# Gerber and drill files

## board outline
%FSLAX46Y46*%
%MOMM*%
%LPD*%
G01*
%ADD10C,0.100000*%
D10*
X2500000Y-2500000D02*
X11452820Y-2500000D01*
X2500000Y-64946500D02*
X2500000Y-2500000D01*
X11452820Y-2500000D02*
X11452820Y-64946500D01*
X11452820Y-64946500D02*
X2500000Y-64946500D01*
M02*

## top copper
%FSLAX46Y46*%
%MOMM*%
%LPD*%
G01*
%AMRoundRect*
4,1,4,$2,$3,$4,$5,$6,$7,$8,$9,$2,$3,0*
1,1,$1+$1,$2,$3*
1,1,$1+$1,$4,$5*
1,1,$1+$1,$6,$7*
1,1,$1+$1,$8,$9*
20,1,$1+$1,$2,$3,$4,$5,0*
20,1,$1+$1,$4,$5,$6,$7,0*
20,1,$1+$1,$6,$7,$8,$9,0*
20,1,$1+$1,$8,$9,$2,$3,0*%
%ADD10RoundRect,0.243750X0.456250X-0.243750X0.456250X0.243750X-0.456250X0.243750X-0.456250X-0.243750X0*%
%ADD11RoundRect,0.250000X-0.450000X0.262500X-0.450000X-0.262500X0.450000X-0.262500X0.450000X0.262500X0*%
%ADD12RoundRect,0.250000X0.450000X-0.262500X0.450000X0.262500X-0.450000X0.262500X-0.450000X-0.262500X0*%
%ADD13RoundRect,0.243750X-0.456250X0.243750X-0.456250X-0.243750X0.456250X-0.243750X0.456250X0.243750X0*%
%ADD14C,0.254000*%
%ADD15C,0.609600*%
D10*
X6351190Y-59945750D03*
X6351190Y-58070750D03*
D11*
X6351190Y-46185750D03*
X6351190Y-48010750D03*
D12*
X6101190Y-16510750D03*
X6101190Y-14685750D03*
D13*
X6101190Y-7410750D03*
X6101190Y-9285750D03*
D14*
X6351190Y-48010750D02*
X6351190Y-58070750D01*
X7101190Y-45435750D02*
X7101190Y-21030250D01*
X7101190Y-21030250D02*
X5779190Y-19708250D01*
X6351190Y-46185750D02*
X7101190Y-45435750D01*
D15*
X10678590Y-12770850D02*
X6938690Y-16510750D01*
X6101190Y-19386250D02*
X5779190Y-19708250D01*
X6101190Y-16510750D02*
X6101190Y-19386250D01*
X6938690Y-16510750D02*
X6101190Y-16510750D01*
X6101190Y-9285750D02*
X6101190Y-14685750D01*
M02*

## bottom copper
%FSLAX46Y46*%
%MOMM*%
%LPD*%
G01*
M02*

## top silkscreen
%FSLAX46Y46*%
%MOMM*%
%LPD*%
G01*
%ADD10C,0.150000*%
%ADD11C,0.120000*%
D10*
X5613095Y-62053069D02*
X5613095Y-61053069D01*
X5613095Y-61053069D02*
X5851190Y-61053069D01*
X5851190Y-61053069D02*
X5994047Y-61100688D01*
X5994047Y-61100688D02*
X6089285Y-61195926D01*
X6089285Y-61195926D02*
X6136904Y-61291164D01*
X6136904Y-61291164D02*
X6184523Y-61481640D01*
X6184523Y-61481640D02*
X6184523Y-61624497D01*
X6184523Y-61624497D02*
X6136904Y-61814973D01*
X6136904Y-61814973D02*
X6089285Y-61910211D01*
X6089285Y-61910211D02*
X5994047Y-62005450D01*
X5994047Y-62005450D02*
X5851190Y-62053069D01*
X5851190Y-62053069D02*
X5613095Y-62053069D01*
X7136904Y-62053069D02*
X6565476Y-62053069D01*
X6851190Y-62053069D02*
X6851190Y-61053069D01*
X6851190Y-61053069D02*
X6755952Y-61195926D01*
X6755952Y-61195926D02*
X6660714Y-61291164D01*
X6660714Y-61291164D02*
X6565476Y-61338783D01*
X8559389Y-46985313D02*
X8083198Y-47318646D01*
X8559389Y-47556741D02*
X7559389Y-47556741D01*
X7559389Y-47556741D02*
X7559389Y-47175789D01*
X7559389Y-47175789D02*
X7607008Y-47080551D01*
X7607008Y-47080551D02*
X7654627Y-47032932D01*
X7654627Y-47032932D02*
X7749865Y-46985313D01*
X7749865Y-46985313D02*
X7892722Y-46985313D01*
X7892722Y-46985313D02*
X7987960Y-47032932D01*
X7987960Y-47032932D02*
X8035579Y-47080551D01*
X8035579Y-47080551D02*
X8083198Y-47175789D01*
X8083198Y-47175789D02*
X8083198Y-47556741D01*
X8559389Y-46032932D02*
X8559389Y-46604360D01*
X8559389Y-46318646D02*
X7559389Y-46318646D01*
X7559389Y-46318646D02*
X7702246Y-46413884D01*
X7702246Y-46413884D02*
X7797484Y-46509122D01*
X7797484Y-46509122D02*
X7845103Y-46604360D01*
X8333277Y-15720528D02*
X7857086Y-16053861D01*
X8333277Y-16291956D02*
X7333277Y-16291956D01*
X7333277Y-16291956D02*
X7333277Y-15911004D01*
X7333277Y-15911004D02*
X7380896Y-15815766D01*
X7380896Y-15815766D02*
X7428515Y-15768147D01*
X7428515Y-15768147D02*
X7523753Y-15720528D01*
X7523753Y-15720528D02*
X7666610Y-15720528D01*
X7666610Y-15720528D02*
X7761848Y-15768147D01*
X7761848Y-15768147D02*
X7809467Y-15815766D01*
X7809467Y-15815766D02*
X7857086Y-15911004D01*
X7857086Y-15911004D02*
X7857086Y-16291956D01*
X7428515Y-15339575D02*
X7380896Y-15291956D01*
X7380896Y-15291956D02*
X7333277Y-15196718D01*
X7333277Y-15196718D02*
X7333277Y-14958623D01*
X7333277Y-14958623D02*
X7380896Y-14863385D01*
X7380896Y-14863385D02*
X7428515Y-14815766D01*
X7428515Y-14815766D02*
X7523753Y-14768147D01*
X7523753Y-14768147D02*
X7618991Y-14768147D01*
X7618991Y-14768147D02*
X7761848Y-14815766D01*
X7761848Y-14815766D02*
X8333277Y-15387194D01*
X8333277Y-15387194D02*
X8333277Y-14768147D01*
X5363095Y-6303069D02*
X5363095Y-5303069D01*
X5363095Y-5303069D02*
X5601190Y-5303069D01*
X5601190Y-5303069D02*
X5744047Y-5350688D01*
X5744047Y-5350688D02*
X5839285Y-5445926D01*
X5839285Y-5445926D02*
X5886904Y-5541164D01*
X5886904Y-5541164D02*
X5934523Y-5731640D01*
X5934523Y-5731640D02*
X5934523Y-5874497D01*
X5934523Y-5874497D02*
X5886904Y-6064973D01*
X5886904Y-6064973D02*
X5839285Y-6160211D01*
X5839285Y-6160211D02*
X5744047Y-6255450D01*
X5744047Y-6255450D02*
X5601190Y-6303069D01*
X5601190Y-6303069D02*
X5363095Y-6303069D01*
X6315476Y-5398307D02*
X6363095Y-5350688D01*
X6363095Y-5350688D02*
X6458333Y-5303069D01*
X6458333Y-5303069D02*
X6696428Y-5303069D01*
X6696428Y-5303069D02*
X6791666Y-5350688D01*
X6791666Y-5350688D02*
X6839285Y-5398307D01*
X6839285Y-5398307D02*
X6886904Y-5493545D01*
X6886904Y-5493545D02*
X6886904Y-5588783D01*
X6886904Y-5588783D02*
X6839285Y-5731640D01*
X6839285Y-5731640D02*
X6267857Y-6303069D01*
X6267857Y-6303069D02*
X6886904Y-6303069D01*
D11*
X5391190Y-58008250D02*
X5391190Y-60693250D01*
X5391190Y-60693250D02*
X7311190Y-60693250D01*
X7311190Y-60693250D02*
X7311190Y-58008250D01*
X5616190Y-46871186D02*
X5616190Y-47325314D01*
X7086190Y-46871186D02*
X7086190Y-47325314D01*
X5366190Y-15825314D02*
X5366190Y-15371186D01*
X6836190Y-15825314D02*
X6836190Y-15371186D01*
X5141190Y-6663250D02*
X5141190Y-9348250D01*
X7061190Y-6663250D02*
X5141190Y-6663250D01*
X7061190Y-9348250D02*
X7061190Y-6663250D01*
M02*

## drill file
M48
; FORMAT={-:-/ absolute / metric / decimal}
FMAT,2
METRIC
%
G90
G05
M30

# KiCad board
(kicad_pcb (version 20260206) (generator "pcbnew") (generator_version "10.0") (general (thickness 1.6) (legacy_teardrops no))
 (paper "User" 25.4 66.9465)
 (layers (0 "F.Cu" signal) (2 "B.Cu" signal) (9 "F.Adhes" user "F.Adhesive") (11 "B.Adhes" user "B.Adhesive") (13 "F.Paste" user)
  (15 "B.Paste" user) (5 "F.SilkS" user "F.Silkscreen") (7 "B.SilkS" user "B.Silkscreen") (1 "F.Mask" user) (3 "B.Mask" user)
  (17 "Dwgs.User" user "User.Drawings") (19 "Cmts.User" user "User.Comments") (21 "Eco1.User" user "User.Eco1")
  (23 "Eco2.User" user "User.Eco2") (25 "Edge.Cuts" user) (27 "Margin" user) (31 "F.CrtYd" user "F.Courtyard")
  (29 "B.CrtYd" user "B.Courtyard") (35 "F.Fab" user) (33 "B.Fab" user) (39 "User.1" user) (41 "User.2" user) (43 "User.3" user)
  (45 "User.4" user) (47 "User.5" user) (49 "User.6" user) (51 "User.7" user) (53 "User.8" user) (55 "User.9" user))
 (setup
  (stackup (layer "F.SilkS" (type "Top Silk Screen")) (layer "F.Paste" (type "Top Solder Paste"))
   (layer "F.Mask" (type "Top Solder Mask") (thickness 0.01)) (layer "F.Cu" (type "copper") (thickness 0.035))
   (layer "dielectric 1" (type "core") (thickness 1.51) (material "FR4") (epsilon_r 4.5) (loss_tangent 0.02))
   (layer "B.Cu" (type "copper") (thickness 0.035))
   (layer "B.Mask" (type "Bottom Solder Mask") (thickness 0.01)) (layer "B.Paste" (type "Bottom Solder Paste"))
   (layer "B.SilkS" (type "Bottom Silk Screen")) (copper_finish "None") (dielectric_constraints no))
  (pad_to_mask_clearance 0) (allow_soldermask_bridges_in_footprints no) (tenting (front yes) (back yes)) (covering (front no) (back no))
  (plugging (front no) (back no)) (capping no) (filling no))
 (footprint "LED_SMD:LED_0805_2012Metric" (layer "F.Cu") (at 6.35119 59.00825 90)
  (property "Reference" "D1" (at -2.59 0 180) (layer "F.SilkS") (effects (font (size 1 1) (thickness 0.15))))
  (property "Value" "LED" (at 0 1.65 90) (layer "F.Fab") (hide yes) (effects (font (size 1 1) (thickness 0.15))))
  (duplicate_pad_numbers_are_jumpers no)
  (fp_line (start 1 -0.96) (end -1.685 -0.96) (stroke (width 0.12) (type solid)) (layer "F.SilkS"))
  (fp_line (start -1.685 -0.96) (end -1.685 0.96) (stroke (width 0.12) (type solid)) (layer "F.SilkS"))
  (fp_line (start -1.685 0.96) (end 1 0.96) (stroke (width 0.12) (type solid)) (layer "F.SilkS"))
  (pad "1" smd roundrect (at -0.9375 0 90) (size 0.975 1.4) (layers "F.Cu" "F.Mask" "F.Paste") (roundrect_rratio 0.25) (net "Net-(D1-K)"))
  (pad "2" smd roundrect (at 0.9375 0 90) (size 0.975 1.4) (layers "F.Cu" "F.Mask" "F.Paste") (roundrect_rratio 0.25) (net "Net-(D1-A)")))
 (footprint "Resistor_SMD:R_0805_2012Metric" (layer "F.Cu") (at 6.35119 47.09825 -90)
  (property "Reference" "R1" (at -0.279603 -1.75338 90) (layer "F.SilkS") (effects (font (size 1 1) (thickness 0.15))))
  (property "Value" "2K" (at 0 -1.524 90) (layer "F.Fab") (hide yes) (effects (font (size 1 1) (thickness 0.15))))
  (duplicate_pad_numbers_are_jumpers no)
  (fp_line (start -0.227064 0.735) (end 0.227064 0.735) (stroke (width 0.12) (type solid)) (layer "F.SilkS"))
  (fp_line (start -0.227064 -0.735) (end 0.227064 -0.735) (stroke (width 0.12) (type solid)) (layer "F.SilkS"))
  (pad "1" smd roundrect (at -0.9125 0 270) (size 1.025 1.4) (layers "F.Cu" "F.Mask" "F.Paste") (roundrect_rratio 0.243902439) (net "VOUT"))
  (pad "2" smd roundrect (at 0.9125 0 270) (size 1.025 1.4) (layers "F.Cu" "F.Mask" "F.Paste") (roundrect_rratio 0.243902439)
   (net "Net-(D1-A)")))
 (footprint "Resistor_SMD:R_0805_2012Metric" (layer "F.Cu") (at 6.10119 15.59825 90)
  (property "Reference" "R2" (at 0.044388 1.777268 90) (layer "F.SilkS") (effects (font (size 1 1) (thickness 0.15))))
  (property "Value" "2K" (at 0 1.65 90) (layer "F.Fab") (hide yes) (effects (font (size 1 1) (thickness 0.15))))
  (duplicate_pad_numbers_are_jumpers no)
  (fp_line (start -0.227064 -0.735) (end 0.227064 -0.735) (stroke (width 0.12) (type solid)) (layer "F.SilkS"))
  (fp_line (start -0.227064 0.735) (end 0.227064 0.735) (stroke (width 0.12) (type solid)) (layer "F.SilkS"))
  (pad "1" smd roundrect (at -0.9125 0 90) (size 1.025 1.4) (layers "F.Cu" "F.Mask" "F.Paste") (roundrect_rratio 0.243902439) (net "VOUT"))
  (pad "2" smd roundrect (at 0.9125 0 90) (size 1.025 1.4) (layers "F.Cu" "F.Mask" "F.Paste") (roundrect_rratio 0.243902439)
   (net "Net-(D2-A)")))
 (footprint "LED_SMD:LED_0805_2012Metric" (layer "F.Cu") (at 6.10119 8.34825 -90)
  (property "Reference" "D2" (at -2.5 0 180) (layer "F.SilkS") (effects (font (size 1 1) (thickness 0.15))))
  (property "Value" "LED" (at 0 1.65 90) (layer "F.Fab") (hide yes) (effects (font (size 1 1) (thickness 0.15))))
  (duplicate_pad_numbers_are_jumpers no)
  (fp_line (start -1.685 0.96) (end 1 0.96) (stroke (width 0.12) (type solid)) (layer "F.SilkS"))
  (fp_line (start -1.685 -0.96) (end -1.685 0.96) (stroke (width 0.12) (type solid)) (layer "F.SilkS"))
  (fp_line (start 1 -0.96) (end -1.685 -0.96) (stroke (width 0.12) (type solid)) (layer "F.SilkS"))
  (pad "1" smd roundrect (at -0.9375 0 270) (size 0.975 1.4) (layers "F.Cu" "F.Mask" "F.Paste") (roundrect_rratio 0.25) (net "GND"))
  (pad "2" smd roundrect (at 0.9375 0 270) (size 0.975 1.4) (layers "F.Cu" "F.Mask" "F.Paste") (roundrect_rratio 0.25) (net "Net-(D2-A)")))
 (gr_line (start 2.5 2.5) (end 11.45282 2.5) (stroke (width 0.1) (type default)) (layer "Edge.Cuts"))
 (gr_line (start 2.5 64.9465) (end 2.5 2.5) (stroke (width 0.1) (type default)) (layer "Edge.Cuts"))
 (gr_line (start 11.45282 2.5) (end 11.45282 64.9465) (stroke (width 0.1) (type default)) (layer "Edge.Cuts"))
 (gr_line (start 11.45282 64.9465) (end 2.5 64.9465) (stroke (width 0.1) (type default)) (layer "Edge.Cuts"))
 (segment (start 6.35119 48.01075) (end 6.35119 58.07075) (width 0.254) (layer "F.Cu") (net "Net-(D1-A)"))
 (segment (start 7.10119 45.43575) (end 7.10119 21.03025) (width 0.254) (layer "F.Cu") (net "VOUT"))
 (segment (start 7.10119 21.03025) (end 5.77919 19.70825) (width 0.254) (layer "F.Cu") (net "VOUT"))
 (segment (start 6.35119 46.18575) (end 7.10119 45.43575) (width 0.254) (layer "F.Cu") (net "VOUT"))
 (segment (start 10.67859 12.77085) (end 6.93869 16.51075) (width 0.6096) (layer "F.Cu") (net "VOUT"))
 (segment (start 6.10119 19.38625) (end 5.77919 19.70825) (width 0.6096) (layer "F.Cu") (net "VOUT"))
 (segment (start 6.10119 16.51075) (end 6.10119 19.38625) (width 0.6096) (layer "F.Cu") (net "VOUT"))
 (segment (start 6.93869 16.51075) (end 6.10119 16.51075) (width 0.6096) (layer "F.Cu") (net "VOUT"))
 (segment (start 6.10119 9.28575) (end 6.10119 14.68575) (width 0.6096) (layer "F.Cu") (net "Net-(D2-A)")))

